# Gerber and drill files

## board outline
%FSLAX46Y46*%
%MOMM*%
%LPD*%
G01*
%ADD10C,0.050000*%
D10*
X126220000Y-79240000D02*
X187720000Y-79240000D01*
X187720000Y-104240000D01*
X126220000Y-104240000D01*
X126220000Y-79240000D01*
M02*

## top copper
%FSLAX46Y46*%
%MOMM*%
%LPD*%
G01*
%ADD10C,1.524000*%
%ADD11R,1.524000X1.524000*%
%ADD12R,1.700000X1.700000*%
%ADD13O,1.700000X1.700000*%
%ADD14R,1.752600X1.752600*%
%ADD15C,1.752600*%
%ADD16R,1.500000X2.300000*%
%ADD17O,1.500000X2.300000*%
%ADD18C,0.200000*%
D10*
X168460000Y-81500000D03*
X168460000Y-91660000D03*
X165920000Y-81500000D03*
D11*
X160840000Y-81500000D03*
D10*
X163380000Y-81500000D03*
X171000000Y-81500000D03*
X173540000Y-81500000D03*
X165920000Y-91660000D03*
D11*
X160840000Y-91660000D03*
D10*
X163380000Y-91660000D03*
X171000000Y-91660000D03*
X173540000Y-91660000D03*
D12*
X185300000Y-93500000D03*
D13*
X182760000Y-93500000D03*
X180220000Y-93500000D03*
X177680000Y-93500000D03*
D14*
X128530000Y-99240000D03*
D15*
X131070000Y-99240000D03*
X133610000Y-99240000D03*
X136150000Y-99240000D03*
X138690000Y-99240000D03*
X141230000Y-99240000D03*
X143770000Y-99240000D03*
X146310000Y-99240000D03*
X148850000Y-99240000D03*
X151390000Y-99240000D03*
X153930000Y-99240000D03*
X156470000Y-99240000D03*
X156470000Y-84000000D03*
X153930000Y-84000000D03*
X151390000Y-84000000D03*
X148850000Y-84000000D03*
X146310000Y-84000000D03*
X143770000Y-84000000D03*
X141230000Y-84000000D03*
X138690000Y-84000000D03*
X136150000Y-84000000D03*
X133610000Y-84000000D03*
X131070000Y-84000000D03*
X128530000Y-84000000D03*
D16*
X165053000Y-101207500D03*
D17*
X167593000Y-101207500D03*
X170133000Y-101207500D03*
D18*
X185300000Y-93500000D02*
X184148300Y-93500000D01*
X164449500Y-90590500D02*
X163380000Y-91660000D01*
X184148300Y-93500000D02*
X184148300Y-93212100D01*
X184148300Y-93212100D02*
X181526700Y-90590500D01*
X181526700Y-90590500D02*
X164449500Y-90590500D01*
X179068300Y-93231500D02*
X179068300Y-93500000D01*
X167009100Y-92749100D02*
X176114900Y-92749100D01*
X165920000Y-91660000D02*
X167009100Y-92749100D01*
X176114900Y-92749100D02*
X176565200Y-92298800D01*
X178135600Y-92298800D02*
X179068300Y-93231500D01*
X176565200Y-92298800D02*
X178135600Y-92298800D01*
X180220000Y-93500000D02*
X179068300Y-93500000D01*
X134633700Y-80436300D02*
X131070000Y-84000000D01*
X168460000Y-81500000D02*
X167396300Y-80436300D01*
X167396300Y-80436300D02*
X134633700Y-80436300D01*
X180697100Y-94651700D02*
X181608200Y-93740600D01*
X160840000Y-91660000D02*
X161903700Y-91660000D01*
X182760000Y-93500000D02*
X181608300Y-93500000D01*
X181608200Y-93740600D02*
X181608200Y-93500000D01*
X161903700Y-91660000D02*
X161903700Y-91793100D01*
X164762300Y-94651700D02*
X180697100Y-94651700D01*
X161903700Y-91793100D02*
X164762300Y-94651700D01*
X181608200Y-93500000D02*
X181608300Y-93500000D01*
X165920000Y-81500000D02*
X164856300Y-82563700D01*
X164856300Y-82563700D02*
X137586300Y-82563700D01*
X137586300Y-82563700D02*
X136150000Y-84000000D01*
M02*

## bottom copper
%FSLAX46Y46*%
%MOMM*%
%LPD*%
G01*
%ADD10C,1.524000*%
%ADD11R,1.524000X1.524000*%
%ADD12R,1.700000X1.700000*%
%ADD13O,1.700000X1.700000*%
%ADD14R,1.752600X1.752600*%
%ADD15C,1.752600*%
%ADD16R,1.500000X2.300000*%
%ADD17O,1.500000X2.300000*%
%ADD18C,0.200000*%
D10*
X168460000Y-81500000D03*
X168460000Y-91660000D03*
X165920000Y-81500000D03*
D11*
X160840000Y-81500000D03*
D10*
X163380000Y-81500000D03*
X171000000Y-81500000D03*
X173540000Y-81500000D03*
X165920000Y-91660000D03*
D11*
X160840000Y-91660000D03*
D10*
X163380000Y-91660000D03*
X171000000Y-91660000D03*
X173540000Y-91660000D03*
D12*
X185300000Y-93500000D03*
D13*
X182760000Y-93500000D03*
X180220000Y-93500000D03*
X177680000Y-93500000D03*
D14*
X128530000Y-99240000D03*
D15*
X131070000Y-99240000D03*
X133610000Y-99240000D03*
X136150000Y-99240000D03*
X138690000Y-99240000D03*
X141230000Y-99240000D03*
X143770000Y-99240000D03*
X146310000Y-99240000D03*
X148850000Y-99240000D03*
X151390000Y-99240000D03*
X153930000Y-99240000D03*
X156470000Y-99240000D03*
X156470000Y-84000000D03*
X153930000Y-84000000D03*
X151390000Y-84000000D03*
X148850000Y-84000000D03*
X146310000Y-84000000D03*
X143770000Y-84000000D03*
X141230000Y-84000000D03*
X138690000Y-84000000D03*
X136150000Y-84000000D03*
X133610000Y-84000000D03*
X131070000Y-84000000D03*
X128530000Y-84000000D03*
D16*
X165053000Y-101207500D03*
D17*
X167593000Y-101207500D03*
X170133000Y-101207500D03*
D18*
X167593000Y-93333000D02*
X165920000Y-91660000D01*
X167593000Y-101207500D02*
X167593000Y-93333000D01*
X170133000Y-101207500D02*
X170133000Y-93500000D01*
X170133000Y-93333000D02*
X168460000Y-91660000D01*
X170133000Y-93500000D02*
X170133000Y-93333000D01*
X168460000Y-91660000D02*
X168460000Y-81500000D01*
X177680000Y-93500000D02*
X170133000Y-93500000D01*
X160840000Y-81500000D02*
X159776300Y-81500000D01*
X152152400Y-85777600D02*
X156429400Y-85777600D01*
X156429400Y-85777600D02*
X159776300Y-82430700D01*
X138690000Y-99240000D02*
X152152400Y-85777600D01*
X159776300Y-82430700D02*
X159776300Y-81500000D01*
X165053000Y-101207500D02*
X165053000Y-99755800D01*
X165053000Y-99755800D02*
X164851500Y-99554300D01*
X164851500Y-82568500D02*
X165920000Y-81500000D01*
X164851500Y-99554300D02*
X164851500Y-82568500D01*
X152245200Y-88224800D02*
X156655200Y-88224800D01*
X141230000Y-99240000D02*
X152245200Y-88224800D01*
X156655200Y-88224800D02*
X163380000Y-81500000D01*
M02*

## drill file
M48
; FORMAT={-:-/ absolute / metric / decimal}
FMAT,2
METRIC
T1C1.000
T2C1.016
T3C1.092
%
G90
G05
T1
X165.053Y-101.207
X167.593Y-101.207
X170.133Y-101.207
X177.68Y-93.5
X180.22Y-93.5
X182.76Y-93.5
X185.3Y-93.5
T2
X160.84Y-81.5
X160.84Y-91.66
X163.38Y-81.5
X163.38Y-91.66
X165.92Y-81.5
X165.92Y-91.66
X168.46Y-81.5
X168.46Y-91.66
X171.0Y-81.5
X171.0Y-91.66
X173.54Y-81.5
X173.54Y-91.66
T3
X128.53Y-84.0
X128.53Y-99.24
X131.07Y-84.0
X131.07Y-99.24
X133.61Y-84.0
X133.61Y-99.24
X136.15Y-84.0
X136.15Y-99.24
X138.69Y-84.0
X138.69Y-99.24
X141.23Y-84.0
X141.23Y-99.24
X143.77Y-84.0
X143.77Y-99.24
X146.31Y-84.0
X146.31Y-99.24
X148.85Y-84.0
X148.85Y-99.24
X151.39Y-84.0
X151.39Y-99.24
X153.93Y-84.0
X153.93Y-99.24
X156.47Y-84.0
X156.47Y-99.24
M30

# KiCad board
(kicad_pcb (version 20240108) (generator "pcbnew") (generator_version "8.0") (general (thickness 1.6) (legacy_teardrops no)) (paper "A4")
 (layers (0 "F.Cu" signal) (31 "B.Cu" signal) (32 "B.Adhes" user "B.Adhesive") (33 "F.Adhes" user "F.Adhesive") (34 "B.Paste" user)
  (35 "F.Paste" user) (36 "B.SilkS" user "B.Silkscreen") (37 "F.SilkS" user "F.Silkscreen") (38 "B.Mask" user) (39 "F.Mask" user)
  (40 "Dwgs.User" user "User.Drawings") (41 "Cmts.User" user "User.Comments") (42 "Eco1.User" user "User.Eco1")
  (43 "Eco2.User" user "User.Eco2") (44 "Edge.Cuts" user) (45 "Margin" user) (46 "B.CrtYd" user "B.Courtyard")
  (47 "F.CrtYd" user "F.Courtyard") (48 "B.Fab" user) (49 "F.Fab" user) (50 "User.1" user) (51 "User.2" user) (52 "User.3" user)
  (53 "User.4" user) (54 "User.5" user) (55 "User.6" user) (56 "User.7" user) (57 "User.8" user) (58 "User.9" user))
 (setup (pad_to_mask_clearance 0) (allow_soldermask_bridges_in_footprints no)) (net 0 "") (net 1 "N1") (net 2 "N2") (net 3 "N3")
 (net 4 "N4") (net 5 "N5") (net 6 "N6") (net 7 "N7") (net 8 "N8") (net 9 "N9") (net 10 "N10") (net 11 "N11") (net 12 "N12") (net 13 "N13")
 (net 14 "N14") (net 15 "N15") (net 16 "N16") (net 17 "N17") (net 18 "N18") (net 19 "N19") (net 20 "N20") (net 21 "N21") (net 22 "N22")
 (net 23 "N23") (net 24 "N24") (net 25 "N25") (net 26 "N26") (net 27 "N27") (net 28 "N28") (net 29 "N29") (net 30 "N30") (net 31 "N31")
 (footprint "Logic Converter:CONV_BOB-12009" (layer "F.Cu") (at 167.19 86.58 90)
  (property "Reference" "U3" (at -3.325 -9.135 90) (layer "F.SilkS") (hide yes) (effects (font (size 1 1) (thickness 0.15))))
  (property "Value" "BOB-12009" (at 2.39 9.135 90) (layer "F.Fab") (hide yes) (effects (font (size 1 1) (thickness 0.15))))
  (pad "GND_1" thru_hole circle (at 5.08 1.27 90) (size 1.524 1.524) (drill 1.016) (layers "*.Cu" "*.Mask") (remove_unused_layers no)
   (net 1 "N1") (solder_mask_margin 0.102))
  (pad "GND_2" thru_hole circle (at -5.08 1.27 90) (size 1.524 1.524) (drill 1.016) (layers "*.Cu" "*.Mask") (remove_unused_layers no)
   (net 1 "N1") (solder_mask_margin 0.102))
  (pad "HV" thru_hole circle (at 5.08 -1.27 90) (size 1.524 1.524) (drill 1.016) (layers "*.Cu" "*.Mask") (remove_unused_layers no)
   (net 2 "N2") (solder_mask_margin 0.102))
  (pad "HV1" thru_hole rect (at 5.08 -6.35 90) (size 1.524 1.524) (drill 1.016) (layers "*.Cu" "*.Mask") (remove_unused_layers no)
   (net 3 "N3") (solder_mask_margin 0.102))
  (pad "HV2" thru_hole circle (at 5.08 -3.81 90) (size 1.524 1.524) (drill 1.016) (layers "*.Cu" "*.Mask") (remove_unused_layers no)
   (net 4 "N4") (solder_mask_margin 0.102))
  (pad "HV3" thru_hole circle (at 5.08 3.81 90) (size 1.524 1.524) (drill 1.016) (layers "*.Cu" "*.Mask") (remove_unused_layers no)
   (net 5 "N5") (solder_mask_margin 0.102))
  (pad "HV4" thru_hole circle (at 5.08 6.35 90) (size 1.524 1.524) (drill 1.016) (layers "*.Cu" "*.Mask") (remove_unused_layers no)
   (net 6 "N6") (solder_mask_margin 0.102))
  (pad "LV" thru_hole circle (at -5.08 -1.27 90) (size 1.524 1.524) (drill 1.016) (layers "*.Cu" "*.Mask") (remove_unused_layers no)
   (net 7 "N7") (solder_mask_margin 0.102))
  (pad "LV1" thru_hole rect (at -5.08 -6.35 90) (size 1.524 1.524) (drill 1.016) (layers "*.Cu" "*.Mask") (remove_unused_layers no)
   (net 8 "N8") (solder_mask_margin 0.102))
  (pad "LV2" thru_hole circle (at -5.08 -3.81 90) (size 1.524 1.524) (drill 1.016) (layers "*.Cu" "*.Mask") (remove_unused_layers no)
   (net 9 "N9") (solder_mask_margin 0.102))
  (pad "LV3" thru_hole circle (at -5.08 3.81 90) (size 1.524 1.524) (drill 1.016) (layers "*.Cu" "*.Mask") (remove_unused_layers no)
   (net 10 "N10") (solder_mask_margin 0.102))
  (pad "LV4" thru_hole circle (at -5.08 6.35 90) (size 1.524 1.524) (drill 1.016) (layers "*.Cu" "*.Mask") (remove_unused_layers no)
   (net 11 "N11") (solder_mask_margin 0.102)))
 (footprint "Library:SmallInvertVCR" (layer "F.Cu") (at 181.5 85)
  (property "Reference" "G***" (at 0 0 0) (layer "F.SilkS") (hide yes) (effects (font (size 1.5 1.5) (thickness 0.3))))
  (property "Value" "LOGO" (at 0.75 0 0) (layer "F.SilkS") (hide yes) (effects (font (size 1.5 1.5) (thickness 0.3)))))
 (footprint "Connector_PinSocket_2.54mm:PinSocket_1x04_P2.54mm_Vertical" (layer "F.Cu") (at 185.3 93.5 -90)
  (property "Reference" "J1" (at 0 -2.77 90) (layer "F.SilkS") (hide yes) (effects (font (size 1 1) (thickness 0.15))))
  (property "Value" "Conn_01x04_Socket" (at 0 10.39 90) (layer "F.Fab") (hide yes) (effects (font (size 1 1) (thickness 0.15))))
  (pad "1" thru_hole rect (at 0 0 270) (size 1.7 1.7) (drill 1) (layers "*.Cu" "*.Mask") (remove_unused_layers no) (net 9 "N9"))
  (pad "2" thru_hole oval (at 0 2.54 270) (size 1.7 1.7) (drill 1) (layers "*.Cu" "*.Mask") (remove_unused_layers no) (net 8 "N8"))
  (pad "3" thru_hole oval (at 0 5.08 270) (size 1.7 1.7) (drill 1) (layers "*.Cu" "*.Mask") (remove_unused_layers no) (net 7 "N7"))
  (pad "4" thru_hole oval (at 0 7.62 270) (size 1.7 1.7) (drill 1) (layers "*.Cu" "*.Mask") (remove_unused_layers no) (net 1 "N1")))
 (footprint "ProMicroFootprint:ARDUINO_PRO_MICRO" (layer "F.Cu") (at 142.5 91.62)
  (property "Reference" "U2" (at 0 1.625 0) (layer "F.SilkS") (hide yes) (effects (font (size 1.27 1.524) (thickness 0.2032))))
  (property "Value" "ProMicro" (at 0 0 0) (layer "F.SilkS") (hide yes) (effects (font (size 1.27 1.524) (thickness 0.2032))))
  (pad "1" thru_hole rect (at -13.97 7.62) (size 1.7526 1.7526) (drill 1.0922) (layers "*.Cu" "*.SilkS" "*.Mask") (remove_unused_layers no)
   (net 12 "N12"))
  (pad "2" thru_hole circle (at -11.43 7.62) (size 1.7526 1.7526) (drill 1.0922) (layers "*.Cu" "*.SilkS" "*.Mask")
   (remove_unused_layers no) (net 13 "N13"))
  (pad "3" thru_hole circle (at -8.89 7.62) (size 1.7526 1.7526) (drill 1.0922) (layers "*.Cu" "*.SilkS" "*.Mask") (remove_unused_layers no)
   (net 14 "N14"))
  (pad "4" thru_hole circle (at -6.35 7.62) (size 1.7526 1.7526) (drill 1.0922) (layers "*.Cu" "*.SilkS" "*.Mask") (remove_unused_layers no)
   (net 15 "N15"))
  (pad "5" thru_hole circle (at -3.81 7.62) (size 1.7526 1.7526) (drill 1.0922) (layers "*.Cu" "*.SilkS" "*.Mask") (remove_unused_layers no)
   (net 3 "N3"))
  (pad "6" thru_hole circle (at -1.27 7.62) (size 1.7526 1.7526) (drill 1.0922) (layers "*.Cu" "*.SilkS" "*.Mask") (remove_unused_layers no)
   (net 4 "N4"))
  (pad "7" thru_hole circle (at 1.27 7.62) (size 1.7526 1.7526) (drill 1.0922) (layers "*.Cu" "*.SilkS" "*.Mask") (remove_unused_layers no)
   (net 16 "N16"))
  (pad "8" thru_hole circle (at 3.81 7.62) (size 1.7526 1.7526) (drill 1.0922) (layers "*.Cu" "*.SilkS" "*.Mask") (remove_unused_layers no)
   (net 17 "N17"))
  (pad "9" thru_hole circle (at 6.35 7.62) (size 1.7526 1.7526) (drill 1.0922) (layers "*.Cu" "*.SilkS" "*.Mask") (remove_unused_layers no)
   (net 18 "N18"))
  (pad "10" thru_hole circle (at 8.89 7.62) (size 1.7526 1.7526) (drill 1.0922) (layers "*.Cu" "*.SilkS" "*.Mask") (remove_unused_layers no)
   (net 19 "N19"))
  (pad "11" thru_hole circle (at 11.43 7.62) (size 1.7526 1.7526) (drill 1.0922) (layers "*.Cu" "*.SilkS" "*.Mask")
   (remove_unused_layers no) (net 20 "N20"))
  (pad "12" thru_hole circle (at 13.97 7.62) (size 1.7526 1.7526) (drill 1.0922) (layers "*.Cu" "*.SilkS" "*.Mask")
   (remove_unused_layers no) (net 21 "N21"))
  (pad "13" thru_hole circle (at 13.97 -7.62) (size 1.7526 1.7526) (drill 1.0922) (layers "*.Cu" "*.SilkS" "*.Mask")
   (remove_unused_layers no) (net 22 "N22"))
  (pad "14" thru_hole circle (at 11.43 -7.62) (size 1.7526 1.7526) (drill 1.0922) (layers "*.Cu" "*.SilkS" "*.Mask")
   (remove_unused_layers no) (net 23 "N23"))
  (pad "15" thru_hole circle (at 8.89 -7.62) (size 1.7526 1.7526) (drill 1.0922) (layers "*.Cu" "*.SilkS" "*.Mask")
   (remove_unused_layers no) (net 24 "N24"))
  (pad "16" thru_hole circle (at 6.35 -7.62) (size 1.7526 1.7526) (drill 1.0922) (layers "*.Cu" "*.SilkS" "*.Mask")
   (remove_unused_layers no) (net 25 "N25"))
  (pad "17" thru_hole circle (at 3.81 -7.62) (size 1.7526 1.7526) (drill 1.0922) (layers "*.Cu" "*.SilkS" "*.Mask")
   (remove_unused_layers no) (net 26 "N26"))
  (pad "18" thru_hole circle (at 1.27 -7.62) (size 1.7526 1.7526) (drill 1.0922) (layers "*.Cu" "*.SilkS" "*.Mask")
   (remove_unused_layers no) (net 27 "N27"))
  (pad "19" thru_hole circle (at -1.27 -7.62) (size 1.7526 1.7526) (drill 1.0922) (layers "*.Cu" "*.SilkS" "*.Mask")
   (remove_unused_layers no) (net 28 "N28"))
  (pad "20" thru_hole circle (at -3.81 -7.62) (size 1.7526 1.7526) (drill 1.0922) (layers "*.Cu" "*.SilkS" "*.Mask")
   (remove_unused_layers no) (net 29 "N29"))
  (pad "21" thru_hole circle (at -6.35 -7.62) (size 1.7526 1.7526) (drill 1.0922) (layers "*.Cu" "*.SilkS" "*.Mask")
   (remove_unused_layers no) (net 2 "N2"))
  (pad "22" thru_hole circle (at -8.89 -7.62) (size 1.7526 1.7526) (drill 1.0922) (layers "*.Cu" "*.SilkS" "*.Mask")
   (remove_unused_layers no) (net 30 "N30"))
  (pad "23" thru_hole circle (at -11.43 -7.62) (size 1.7526 1.7526) (drill 1.0922) (layers "*.Cu" "*.SilkS" "*.Mask")
   (remove_unused_layers no) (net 1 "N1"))
  (pad "24" thru_hole circle (at -13.97 -7.62) (size 1.7526 1.7526) (drill 1.0922) (layers "*.Cu" "*.SilkS" "*.Mask")
   (remove_unused_layers no) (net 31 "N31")))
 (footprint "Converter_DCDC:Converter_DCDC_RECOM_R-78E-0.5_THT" (layer "F.Cu") (at 165.053 101.2075)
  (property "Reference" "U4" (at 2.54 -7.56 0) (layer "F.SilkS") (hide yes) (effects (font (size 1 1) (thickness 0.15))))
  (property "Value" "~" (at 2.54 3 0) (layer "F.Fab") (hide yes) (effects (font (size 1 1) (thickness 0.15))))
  (pad "1" thru_hole rect (at 0 0) (size 1.5 2.3) (drill 1) (layers "*.Cu" "*.Mask") (remove_unused_layers no) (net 2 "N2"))
  (pad "2" thru_hole oval (at 2.54 0) (size 1.5 2.3) (drill 1) (layers "*.Cu" "*.Mask") (remove_unused_layers no) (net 7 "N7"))
  (pad "3" thru_hole oval (at 5.08 0) (size 1.5 2.3) (drill 1) (layers "*.Cu" "*.Mask") (remove_unused_layers no) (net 1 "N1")))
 (gr_rect (start 126.22 79.24) (end 187.72 104.24) (stroke (width 0.05) (type default)) (fill none) (layer "Edge.Cuts"))
 (segment (start 185.3 93.5) (end 184.1483 93.5) (width 0.2) (layer "F.Cu") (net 9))
 (segment (start 164.4495 90.5905) (end 163.38 91.66) (width 0.2) (layer "F.Cu") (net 9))
 (segment (start 184.1483 93.5) (end 184.1483 93.2121) (width 0.2) (layer "F.Cu") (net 9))
 (segment (start 184.1483 93.2121) (end 181.5267 90.5905) (width 0.2) (layer "F.Cu") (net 9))
 (segment (start 181.5267 90.5905) (end 164.4495 90.5905) (width 0.2) (layer "F.Cu") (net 9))
 (segment (start 179.0683 93.2315) (end 179.0683 93.5) (width 0.2) (layer "F.Cu") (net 7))
 (segment (start 167.0091 92.7491) (end 176.1149 92.7491) (width 0.2) (layer "F.Cu") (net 7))
 (segment (start 165.92 91.66) (end 167.0091 92.7491) (width 0.2) (layer "F.Cu") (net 7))
 (segment (start 176.1149 92.7491) (end 176.5652 92.2988) (width 0.2) (layer "F.Cu") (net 7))
 (segment (start 178.1356 92.2988) (end 179.0683 93.2315) (width 0.2) (layer "F.Cu") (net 7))
 (segment (start 176.5652 92.2988) (end 178.1356 92.2988) (width 0.2) (layer "F.Cu") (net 7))
 (segment (start 180.22 93.5) (end 179.0683 93.5) (width 0.2) (layer "F.Cu") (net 7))
 (segment (start 167.593 93.333) (end 165.92 91.66) (width 0.2) (layer "B.Cu") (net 7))
 (segment (start 167.593 101.2075) (end 167.593 93.333) (width 0.2) (layer "B.Cu") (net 7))
 (segment (start 134.6337 80.4363) (end 131.07 84) (width 0.2) (layer "F.Cu") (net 1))
 (segment (start 168.46 81.5) (end 167.3963 80.4363) (width 0.2) (layer "F.Cu") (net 1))
 (segment (start 167.3963 80.4363) (end 134.6337 80.4363) (width 0.2) (layer "F.Cu") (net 1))
 (segment (start 170.133 101.2075) (end 170.133 93.5) (width 0.2) (layer "B.Cu") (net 1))
 (segment (start 170.133 93.333) (end 168.46 91.66) (width 0.2) (layer "B.Cu") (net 1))
 (segment (start 170.133 93.5) (end 170.133 93.333) (width 0.2) (layer "B.Cu") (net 1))
 (segment (start 168.46 91.66) (end 168.46 81.5) (width 0.2) (layer "B.Cu") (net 1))
 (segment (start 177.68 93.5) (end 170.133 93.5) (width 0.2) (layer "B.Cu") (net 1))
 (segment (start 180.6971 94.6517) (end 181.6082 93.7406) (width 0.2) (layer "F.Cu") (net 8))
 (segment (start 160.84 91.66) (end 161.9037 91.66) (width 0.2) (layer "F.Cu") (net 8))
 (segment (start 182.76 93.5) (end 181.6083 93.5) (width 0.2) (layer "F.Cu") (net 8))
 (segment (start 181.6082 93.7406) (end 181.6082 93.5) (width 0.2) (layer "F.Cu") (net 8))
 (segment (start 161.9037 91.66) (end 161.9037 91.7931) (width 0.2) (layer "F.Cu") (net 8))
 (segment (start 164.7623 94.6517) (end 180.6971 94.6517) (width 0.2) (layer "F.Cu") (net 8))
 (segment (start 161.9037 91.7931) (end 164.7623 94.6517) (width 0.2) (layer "F.Cu") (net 8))
 (segment (start 181.6082 93.5) (end 181.6083 93.5) (width 0.2) (layer "F.Cu") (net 8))
 (segment (start 160.84 81.5) (end 159.7763 81.5) (width 0.2) (layer "B.Cu") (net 3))
 (segment (start 152.1524 85.7776) (end 156.4294 85.7776) (width 0.2) (layer "B.Cu") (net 3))
 (segment (start 156.4294 85.7776) (end 159.7763 82.4307) (width 0.2) (layer "B.Cu") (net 3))
 (segment (start 138.69 99.24) (end 152.1524 85.7776) (width 0.2) (layer "B.Cu") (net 3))
 (segment (start 159.7763 82.4307) (end 159.7763 81.5) (width 0.2) (layer "B.Cu") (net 3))
 (segment (start 165.92 81.5) (end 164.8563 82.5637) (width 0.2) (layer "F.Cu") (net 2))
 (segment (start 164.8563 82.5637) (end 137.5863 82.5637) (width 0.2) (layer "F.Cu") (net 2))
 (segment (start 137.5863 82.5637) (end 136.15 84) (width 0.2) (layer "F.Cu") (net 2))
 (segment (start 165.053 101.2075) (end 165.053 99.7558) (width 0.2) (layer "B.Cu") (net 2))
 (segment (start 165.053 99.7558) (end 164.8515 99.5543) (width 0.2) (layer "B.Cu") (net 2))
 (segment (start 164.8515 82.5685) (end 165.92 81.5) (width 0.2) (layer "B.Cu") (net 2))
 (segment (start 164.8515 99.5543) (end 164.8515 82.5685) (width 0.2) (layer "B.Cu") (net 2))
 (segment (start 152.2452 88.2248) (end 156.6552 88.2248) (width 0.2) (layer "B.Cu") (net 4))
 (segment (start 141.23 99.24) (end 152.2452 88.2248) (width 0.2) (layer "B.Cu") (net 4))
 (segment (start 156.6552 88.2248) (end 163.38 81.5) (width 0.2) (layer "B.Cu") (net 4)))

